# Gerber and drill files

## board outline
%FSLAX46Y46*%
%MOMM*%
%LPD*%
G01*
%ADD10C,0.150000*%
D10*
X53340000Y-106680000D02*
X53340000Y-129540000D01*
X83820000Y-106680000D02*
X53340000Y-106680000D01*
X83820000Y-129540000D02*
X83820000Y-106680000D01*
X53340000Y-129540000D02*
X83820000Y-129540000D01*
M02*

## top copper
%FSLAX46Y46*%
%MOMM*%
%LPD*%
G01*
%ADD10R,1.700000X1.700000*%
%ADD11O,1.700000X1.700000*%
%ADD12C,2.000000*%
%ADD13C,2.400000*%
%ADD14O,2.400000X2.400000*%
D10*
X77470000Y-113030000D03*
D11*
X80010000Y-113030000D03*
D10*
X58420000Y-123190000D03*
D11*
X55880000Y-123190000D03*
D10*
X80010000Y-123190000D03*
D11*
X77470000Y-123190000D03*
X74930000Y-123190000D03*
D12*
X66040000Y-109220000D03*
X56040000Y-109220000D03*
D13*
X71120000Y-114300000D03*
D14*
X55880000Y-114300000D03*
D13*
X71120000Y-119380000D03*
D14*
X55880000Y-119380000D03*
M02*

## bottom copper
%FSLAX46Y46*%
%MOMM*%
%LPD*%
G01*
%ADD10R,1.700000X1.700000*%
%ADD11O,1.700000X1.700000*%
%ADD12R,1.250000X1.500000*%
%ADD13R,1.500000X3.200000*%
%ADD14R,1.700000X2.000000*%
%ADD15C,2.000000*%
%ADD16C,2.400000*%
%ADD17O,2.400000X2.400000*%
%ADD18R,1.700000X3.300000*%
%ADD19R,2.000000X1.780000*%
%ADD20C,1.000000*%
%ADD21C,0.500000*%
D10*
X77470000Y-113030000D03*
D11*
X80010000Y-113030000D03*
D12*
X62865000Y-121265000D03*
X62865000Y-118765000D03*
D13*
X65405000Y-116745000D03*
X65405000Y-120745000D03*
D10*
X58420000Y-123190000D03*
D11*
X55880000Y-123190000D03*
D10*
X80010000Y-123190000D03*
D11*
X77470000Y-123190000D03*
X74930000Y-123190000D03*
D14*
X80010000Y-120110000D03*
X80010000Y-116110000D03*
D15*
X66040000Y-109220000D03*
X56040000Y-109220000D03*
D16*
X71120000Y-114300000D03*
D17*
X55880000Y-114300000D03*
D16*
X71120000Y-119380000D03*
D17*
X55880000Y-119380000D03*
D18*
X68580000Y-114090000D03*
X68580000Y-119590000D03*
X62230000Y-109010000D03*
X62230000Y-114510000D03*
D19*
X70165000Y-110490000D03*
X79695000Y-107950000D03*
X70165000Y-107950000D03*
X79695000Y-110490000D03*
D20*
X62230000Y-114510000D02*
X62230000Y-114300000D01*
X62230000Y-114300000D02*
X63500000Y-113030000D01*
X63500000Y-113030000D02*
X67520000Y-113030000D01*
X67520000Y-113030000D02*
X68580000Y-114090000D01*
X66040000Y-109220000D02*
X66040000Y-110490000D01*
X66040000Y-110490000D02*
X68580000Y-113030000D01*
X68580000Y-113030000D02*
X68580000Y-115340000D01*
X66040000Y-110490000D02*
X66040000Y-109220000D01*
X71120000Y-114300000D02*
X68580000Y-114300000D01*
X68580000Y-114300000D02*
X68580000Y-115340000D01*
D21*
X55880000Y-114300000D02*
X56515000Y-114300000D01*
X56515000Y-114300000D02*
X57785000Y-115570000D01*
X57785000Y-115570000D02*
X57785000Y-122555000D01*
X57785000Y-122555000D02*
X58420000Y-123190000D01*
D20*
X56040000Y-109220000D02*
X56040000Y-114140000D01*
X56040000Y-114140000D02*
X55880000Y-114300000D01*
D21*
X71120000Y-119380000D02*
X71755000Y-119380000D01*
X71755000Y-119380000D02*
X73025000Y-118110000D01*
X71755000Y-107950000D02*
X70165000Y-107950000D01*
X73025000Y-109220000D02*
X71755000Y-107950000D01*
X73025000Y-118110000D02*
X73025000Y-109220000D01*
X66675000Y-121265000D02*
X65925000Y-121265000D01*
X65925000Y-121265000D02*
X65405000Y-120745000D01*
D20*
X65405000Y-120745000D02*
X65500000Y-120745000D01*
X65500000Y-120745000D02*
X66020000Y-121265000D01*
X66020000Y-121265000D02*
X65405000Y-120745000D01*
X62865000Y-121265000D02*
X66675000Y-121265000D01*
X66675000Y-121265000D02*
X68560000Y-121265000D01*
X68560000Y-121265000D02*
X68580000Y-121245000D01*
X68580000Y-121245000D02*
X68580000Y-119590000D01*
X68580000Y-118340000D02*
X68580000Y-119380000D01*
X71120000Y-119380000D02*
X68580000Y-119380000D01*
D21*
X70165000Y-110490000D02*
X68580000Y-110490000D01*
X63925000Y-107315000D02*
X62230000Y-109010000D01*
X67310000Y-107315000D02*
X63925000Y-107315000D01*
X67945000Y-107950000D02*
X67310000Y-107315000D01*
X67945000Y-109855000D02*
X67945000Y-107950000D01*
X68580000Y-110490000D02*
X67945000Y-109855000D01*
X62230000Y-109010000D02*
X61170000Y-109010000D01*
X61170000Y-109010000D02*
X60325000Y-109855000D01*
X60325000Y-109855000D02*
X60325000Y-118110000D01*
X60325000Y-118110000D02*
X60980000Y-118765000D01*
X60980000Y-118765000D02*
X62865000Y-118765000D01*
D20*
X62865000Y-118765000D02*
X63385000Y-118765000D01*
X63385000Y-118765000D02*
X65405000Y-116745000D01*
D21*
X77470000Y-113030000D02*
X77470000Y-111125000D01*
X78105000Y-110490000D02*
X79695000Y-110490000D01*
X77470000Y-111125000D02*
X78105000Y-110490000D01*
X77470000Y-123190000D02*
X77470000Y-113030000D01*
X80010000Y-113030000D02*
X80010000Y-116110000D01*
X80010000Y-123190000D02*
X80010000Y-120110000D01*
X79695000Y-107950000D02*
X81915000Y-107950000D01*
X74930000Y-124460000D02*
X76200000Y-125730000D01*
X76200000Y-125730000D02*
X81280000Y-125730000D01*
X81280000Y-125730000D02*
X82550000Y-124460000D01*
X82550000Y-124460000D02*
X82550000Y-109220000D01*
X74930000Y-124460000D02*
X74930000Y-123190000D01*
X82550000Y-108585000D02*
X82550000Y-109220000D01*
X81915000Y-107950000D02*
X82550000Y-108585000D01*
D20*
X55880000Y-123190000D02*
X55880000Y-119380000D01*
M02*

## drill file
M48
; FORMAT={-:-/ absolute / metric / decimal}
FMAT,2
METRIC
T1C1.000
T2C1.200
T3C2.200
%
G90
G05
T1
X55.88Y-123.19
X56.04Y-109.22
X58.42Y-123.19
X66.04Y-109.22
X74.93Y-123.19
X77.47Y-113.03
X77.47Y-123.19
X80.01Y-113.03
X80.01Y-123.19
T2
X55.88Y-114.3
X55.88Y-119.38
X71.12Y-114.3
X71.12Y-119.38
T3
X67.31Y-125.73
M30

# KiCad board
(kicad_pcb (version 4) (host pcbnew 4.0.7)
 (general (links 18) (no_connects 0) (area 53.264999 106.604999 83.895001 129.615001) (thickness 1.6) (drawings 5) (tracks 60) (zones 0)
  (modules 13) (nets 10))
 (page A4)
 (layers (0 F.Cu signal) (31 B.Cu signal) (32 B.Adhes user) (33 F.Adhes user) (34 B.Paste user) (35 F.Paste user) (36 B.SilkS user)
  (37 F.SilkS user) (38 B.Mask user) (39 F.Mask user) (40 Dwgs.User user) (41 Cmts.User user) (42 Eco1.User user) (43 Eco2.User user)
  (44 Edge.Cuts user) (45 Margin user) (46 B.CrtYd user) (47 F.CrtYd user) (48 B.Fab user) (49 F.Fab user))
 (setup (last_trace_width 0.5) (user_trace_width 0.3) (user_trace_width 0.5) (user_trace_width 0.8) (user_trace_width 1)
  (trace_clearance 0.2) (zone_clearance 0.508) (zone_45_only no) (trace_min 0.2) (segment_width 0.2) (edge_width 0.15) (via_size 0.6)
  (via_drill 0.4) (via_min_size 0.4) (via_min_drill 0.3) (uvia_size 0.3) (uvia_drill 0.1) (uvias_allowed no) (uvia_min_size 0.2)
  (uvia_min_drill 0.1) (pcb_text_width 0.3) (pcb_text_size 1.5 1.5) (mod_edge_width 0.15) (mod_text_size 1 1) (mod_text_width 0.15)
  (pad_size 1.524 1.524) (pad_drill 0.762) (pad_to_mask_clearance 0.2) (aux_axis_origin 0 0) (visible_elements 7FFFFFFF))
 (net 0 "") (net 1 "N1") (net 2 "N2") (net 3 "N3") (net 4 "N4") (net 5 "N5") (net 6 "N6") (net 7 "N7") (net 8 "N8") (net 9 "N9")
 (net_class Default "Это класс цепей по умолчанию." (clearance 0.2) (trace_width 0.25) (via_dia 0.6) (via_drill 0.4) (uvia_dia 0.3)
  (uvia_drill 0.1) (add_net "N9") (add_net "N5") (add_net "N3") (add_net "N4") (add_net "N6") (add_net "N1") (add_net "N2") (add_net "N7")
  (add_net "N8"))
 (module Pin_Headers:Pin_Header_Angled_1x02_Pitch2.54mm (layer F.Cu) (at 77.47 113.03 90)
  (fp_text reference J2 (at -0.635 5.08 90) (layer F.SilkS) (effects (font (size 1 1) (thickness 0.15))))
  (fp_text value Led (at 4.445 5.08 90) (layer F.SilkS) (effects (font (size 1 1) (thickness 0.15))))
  (pad 1 thru_hole rect (at 0 0 90) (size 1.7 1.7) (drill 1) (layers *.Cu *.Mask) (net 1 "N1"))
  (pad 2 thru_hole oval (at 0 2.54 90) (size 1.7 1.7) (drill 1) (layers *.Cu *.Mask) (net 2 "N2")))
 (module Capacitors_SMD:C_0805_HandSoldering (layer B.Cu) (at 62.865 120.015 90)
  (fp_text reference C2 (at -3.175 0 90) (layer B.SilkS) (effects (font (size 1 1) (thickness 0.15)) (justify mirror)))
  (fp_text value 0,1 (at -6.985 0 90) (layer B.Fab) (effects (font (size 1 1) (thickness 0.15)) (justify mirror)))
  (pad 1 smd rect (at -1.25 0 90) (size 1.5 1.25) (layers B.Cu B.Paste B.Mask) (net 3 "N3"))
  (pad 2 smd rect (at 1.25 0 90) (size 1.5 1.25) (layers B.Cu B.Paste B.Mask) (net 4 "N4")))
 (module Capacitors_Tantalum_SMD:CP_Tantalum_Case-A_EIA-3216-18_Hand (layer B.Cu) (at 65.405 118.745 270)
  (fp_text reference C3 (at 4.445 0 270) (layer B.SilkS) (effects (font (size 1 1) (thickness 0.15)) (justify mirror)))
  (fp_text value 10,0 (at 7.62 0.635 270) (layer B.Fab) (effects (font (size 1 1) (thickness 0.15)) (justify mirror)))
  (pad 1 smd rect (at -2 0 270) (size 3.2 1.5) (layers B.Cu B.Paste B.Mask) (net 4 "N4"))
  (pad 2 smd rect (at 2 0 270) (size 3.2 1.5) (layers B.Cu B.Paste B.Mask) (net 3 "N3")))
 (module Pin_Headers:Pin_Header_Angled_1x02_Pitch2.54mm (layer F.Cu) (at 58.42 123.19 270)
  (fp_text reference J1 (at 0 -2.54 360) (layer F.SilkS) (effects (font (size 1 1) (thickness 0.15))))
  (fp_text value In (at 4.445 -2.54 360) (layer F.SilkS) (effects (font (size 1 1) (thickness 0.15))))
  (pad 1 thru_hole rect (at 0 0 270) (size 1.7 1.7) (drill 1) (layers *.Cu *.Mask) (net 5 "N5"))
  (pad 2 thru_hole oval (at 0 2.54 270) (size 1.7 1.7) (drill 1) (layers *.Cu *.Mask) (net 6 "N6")))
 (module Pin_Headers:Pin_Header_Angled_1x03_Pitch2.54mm (layer F.Cu) (at 80.01 123.19 270)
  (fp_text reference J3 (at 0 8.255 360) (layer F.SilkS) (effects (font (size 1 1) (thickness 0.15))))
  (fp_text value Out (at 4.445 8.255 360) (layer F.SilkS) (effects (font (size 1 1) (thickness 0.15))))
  (pad 1 thru_hole rect (at 0 0 270) (size 1.7 1.7) (drill 1) (layers *.Cu *.Mask) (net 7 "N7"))
  (pad 2 thru_hole oval (at 0 2.54 270) (size 1.7 1.7) (drill 1) (layers *.Cu *.Mask) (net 1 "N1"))
  (pad 3 thru_hole oval (at 0 5.08 270) (size 1.7 1.7) (drill 1) (layers *.Cu *.Mask) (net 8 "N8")))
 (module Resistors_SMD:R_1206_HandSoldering (layer B.Cu) (at 80.01 118.11 90)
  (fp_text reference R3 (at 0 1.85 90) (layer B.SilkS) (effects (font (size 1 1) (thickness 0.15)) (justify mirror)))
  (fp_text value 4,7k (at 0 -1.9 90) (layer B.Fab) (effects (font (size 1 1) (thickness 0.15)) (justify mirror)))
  (pad 1 smd rect (at -2 0 90) (size 2 1.7) (layers B.Cu B.Paste B.Mask) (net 7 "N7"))
  (pad 2 smd rect (at 2 0 90) (size 2 1.7) (layers B.Cu B.Paste B.Mask) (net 2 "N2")))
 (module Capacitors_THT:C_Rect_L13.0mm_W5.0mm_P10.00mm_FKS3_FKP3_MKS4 (layer F.Cu) (at 66.04 109.22 180)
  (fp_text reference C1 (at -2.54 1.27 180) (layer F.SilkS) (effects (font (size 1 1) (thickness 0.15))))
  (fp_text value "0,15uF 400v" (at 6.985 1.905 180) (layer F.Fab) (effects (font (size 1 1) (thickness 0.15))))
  (pad 1 thru_hole circle (at 0 0 180) (size 2 2) (drill 1) (layers *.Cu *.Mask) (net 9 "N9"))
  (pad 2 thru_hole circle (at 10 0 180) (size 2 2) (drill 1) (layers *.Cu *.Mask) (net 5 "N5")))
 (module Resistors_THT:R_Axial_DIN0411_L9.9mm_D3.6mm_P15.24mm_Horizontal (layer F.Cu) (at 71.12 114.3 180)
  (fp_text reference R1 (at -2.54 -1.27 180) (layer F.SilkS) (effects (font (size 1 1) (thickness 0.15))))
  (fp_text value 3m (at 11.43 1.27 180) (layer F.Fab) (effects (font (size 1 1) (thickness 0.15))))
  (pad 1 thru_hole circle (at 0 0 180) (size 2.4 2.4) (drill 1.2) (layers *.Cu *.Mask) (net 9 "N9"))
  (pad 2 thru_hole oval (at 15.24 0 180) (size 2.4 2.4) (drill 1.2) (layers *.Cu *.Mask) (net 5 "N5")))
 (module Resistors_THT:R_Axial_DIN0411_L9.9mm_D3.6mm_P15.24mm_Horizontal (layer F.Cu) (at 71.12 119.38 180)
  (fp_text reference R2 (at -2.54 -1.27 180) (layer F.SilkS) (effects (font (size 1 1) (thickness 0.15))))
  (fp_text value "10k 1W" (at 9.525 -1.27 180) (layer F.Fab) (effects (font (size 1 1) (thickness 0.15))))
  (pad 1 thru_hole circle (at 0 0 180) (size 2.4 2.4) (drill 1.2) (layers *.Cu *.Mask) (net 3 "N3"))
  (pad 2 thru_hole oval (at 15.24 0 180) (size 2.4 2.4) (drill 1.2) (layers *.Cu *.Mask) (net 6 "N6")))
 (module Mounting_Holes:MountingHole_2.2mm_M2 (layer F.Cu) (at 67.31 125.73)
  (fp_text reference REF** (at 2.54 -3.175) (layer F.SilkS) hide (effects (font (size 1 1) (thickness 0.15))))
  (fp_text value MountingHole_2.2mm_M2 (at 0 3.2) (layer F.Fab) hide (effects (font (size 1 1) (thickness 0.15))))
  (pad 1 np_thru_hole circle (at 0 0) (size 2.2 2.2) (drill 2.2) (layers *.Cu *.Mask)))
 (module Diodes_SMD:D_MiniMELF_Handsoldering (layer B.Cu) (at 68.58 116.84 270)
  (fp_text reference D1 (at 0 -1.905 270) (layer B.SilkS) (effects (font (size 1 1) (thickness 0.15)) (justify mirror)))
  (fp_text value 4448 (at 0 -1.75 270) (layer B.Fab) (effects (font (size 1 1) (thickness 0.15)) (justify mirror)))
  (pad 1 smd rect (at -2.75 0 270) (size 3.3 1.7) (layers B.Cu B.Paste B.Mask) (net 9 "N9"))
  (pad 2 smd rect (at 2.75 0 270) (size 3.3 1.7) (layers B.Cu B.Paste B.Mask) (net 3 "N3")))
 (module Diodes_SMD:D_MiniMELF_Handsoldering (layer B.Cu) (at 62.23 111.76 270)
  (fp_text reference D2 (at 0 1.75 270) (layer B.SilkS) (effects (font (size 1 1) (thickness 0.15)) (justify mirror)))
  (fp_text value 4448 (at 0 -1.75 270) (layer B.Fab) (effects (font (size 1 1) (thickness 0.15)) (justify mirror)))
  (pad 1 smd rect (at -2.75 0 270) (size 3.3 1.7) (layers B.Cu B.Paste B.Mask) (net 4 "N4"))
  (pad 2 smd rect (at 2.75 0 270) (size 3.3 1.7) (layers B.Cu B.Paste B.Mask) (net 9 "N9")))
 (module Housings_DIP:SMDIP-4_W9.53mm (layer B.Cu) (at 74.93 109.22)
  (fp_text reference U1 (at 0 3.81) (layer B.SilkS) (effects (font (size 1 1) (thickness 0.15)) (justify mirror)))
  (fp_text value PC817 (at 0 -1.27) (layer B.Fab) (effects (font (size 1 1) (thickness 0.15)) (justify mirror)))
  (pad 1 smd rect (at -4.765 1.27) (size 2 1.78) (layers B.Cu B.Paste B.Mask) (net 4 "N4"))
  (pad 3 smd rect (at 4.765 -1.27) (size 2 1.78) (layers B.Cu B.Paste B.Mask) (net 8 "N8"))
  (pad 2 smd rect (at -4.765 -1.27) (size 2 1.78) (layers B.Cu B.Paste B.Mask) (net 3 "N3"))
  (pad 4 smd rect (at 4.765 1.27) (size 2 1.78) (layers B.Cu B.Paste B.Mask) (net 1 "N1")))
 (gr_line (start 53.34 106.68) (end 53.34 129.54) (angle 90) (layer Edge.Cuts) (width 0.15))
 (gr_line (start 83.82 106.68) (end 53.34 106.68) (angle 90) (layer Edge.Cuts) (width 0.15))
 (gr_line (start 83.82 129.54) (end 83.82 106.68) (angle 90) (layer Edge.Cuts) (width 0.15))
 (gr_line (start 53.34 129.54) (end 83.82 129.54) (angle 90) (layer Edge.Cuts) (width 0.15))
 (segment (start 62.23 114.51) (end 62.23 114.3) (width 1) (layer B.Cu) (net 9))
 (segment (start 62.23 114.3) (end 63.5 113.03) (width 1) (layer B.Cu) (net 9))
 (segment (start 63.5 113.03) (end 67.52 113.03) (width 1) (layer B.Cu) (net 9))
 (segment (start 67.52 113.03) (end 68.58 114.09) (width 1) (layer B.Cu) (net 9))
 (segment (start 66.04 109.22) (end 66.04 110.49) (width 1) (layer B.Cu) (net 9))
 (segment (start 66.04 110.49) (end 68.58 113.03) (width 1) (layer B.Cu) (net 9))
 (segment (start 68.58 113.03) (end 68.58 115.34) (width 1) (layer B.Cu) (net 9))
 (segment (start 66.04 110.49) (end 66.04 109.22) (width 1) (layer B.Cu) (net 9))
 (segment (start 71.12 114.3) (end 68.58 114.3) (width 1) (layer B.Cu) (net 9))
 (segment (start 68.58 114.3) (end 68.58 115.34) (width 1) (layer B.Cu) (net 9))
 (segment (start 55.88 114.3) (end 56.515 114.3) (width 0.5) (layer B.Cu) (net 5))
 (segment (start 56.515 114.3) (end 57.785 115.57) (width 0.5) (layer B.Cu) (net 5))
 (segment (start 57.785 115.57) (end 57.785 122.555) (width 0.5) (layer B.Cu) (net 5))
 (segment (start 57.785 122.555) (end 58.42 123.19) (width 0.5) (layer B.Cu) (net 5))
 (segment (start 56.04 109.22) (end 56.04 114.14) (width 1) (layer B.Cu) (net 5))
 (segment (start 56.04 114.14) (end 55.88 114.3) (width 1) (layer B.Cu) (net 5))
 (segment (start 71.12 119.38) (end 71.755 119.38) (width 0.5) (layer B.Cu) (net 3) (status C00000))
 (segment (start 71.755 119.38) (end 73.025 118.11) (width 0.5) (layer B.Cu) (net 3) (status 400000))
 (segment (start 71.755 107.95) (end 70.165 107.95) (width 0.5) (layer B.Cu) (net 3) (status 800000))
 (segment (start 73.025 109.22) (end 71.755 107.95) (width 0.5) (layer B.Cu) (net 3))
 (segment (start 73.025 118.11) (end 73.025 109.22) (width 0.5) (layer B.Cu) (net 3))
 (segment (start 66.675 121.265) (end 65.925 121.265) (width 0.5) (layer B.Cu) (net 3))
 (segment (start 65.925 121.265) (end 65.405 120.745) (width 0.5) (layer B.Cu) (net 3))
 (segment (start 65.405 120.745) (end 65.5 120.745) (width 1) (layer B.Cu) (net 3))
 (segment (start 65.5 120.745) (end 66.02 121.265) (width 1) (layer B.Cu) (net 3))
 (segment (start 66.02 121.265) (end 65.405 120.745) (width 1) (layer B.Cu) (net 3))
 (segment (start 62.865 121.265) (end 66.675 121.265) (width 1) (layer B.Cu) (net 3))
 (segment (start 66.675 121.265) (end 68.56 121.265) (width 1) (layer B.Cu) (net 3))
 (segment (start 68.56 121.265) (end 68.58 121.245) (width 1) (layer B.Cu) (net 3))
 (segment (start 68.58 121.245) (end 68.58 119.59) (width 1) (layer B.Cu) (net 3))
 (segment (start 68.58 118.34) (end 68.58 119.38) (width 1) (layer B.Cu) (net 3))
 (segment (start 71.12 119.38) (end 68.58 119.38) (width 1) (layer B.Cu) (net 3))
 (segment (start 70.165 110.49) (end 68.58 110.49) (width 0.5) (layer B.Cu) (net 4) (status 400000))
 (segment (start 63.925 107.315) (end 62.23 109.01) (width 0.5) (layer B.Cu) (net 4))
 (segment (start 67.31 107.315) (end 63.925 107.315) (width 0.5) (layer B.Cu) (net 4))
 (segment (start 67.945 107.95) (end 67.31 107.315) (width 0.5) (layer B.Cu) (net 4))
 (segment (start 67.945 109.855) (end 67.945 107.95) (width 0.5) (layer B.Cu) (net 4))
 (segment (start 68.58 110.49) (end 67.945 109.855) (width 0.5) (layer B.Cu) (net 4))
 (segment (start 62.23 109.01) (end 61.17 109.01) (width 0.5) (layer B.Cu) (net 4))
 (segment (start 61.17 109.01) (end 60.325 109.855) (width 0.5) (layer B.Cu) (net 4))
 (segment (start 60.325 109.855) (end 60.325 118.11) (width 0.5) (layer B.Cu) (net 4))
 (segment (start 60.325 118.11) (end 60.98 118.765) (width 0.5) (layer B.Cu) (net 4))
 (segment (start 60.98 118.765) (end 62.865 118.765) (width 0.5) (layer B.Cu) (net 4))
 (segment (start 62.865 118.765) (end 63.385 118.765) (width 1) (layer B.Cu) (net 4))
 (segment (start 63.385 118.765) (end 65.405 116.745) (width 1) (layer B.Cu) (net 4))
 (segment (start 77.47 113.03) (end 77.47 111.125) (width 0.5) (layer B.Cu) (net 1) (status 400000))
 (segment (start 78.105 110.49) (end 79.695 110.49) (width 0.5) (layer B.Cu) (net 1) (status 800000))
 (segment (start 77.47 111.125) (end 78.105 110.49) (width 0.5) (layer B.Cu) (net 1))
 (segment (start 77.47 123.19) (end 77.47 113.03) (width 0.5) (layer B.Cu) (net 1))
 (segment (start 80.01 113.03) (end 80.01 116.11) (width 0.5) (layer B.Cu) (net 2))
 (segment (start 80.01 123.19) (end 80.01 120.11) (width 0.5) (layer B.Cu) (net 7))
 (segment (start 79.695 107.95) (end 81.915 107.95) (width 0.5) (layer B.Cu) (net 8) (status 400000))
 (segment (start 74.93 124.46) (end 76.2 125.73) (width 0.5) (layer B.Cu) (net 8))
 (segment (start 76.2 125.73) (end 81.28 125.73) (width 0.5) (layer B.Cu) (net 8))
 (segment (start 81.28 125.73) (end 82.55 124.46) (width 0.5) (layer B.Cu) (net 8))
 (segment (start 82.55 124.46) (end 82.55 109.22) (width 0.5) (layer B.Cu) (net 8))
 (segment (start 74.93 124.46) (end 74.93 123.19) (width 0.5) (layer B.Cu) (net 8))
 (segment (start 82.55 108.585) (end 82.55 109.22) (width 0.5) (layer B.Cu) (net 8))
 (segment (start 81.915 107.95) (end 82.55 108.585) (width 0.5) (layer B.Cu) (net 8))
 (segment (start 55.88 123.19) (end 55.88 119.38) (width 1) (layer B.Cu) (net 6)))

